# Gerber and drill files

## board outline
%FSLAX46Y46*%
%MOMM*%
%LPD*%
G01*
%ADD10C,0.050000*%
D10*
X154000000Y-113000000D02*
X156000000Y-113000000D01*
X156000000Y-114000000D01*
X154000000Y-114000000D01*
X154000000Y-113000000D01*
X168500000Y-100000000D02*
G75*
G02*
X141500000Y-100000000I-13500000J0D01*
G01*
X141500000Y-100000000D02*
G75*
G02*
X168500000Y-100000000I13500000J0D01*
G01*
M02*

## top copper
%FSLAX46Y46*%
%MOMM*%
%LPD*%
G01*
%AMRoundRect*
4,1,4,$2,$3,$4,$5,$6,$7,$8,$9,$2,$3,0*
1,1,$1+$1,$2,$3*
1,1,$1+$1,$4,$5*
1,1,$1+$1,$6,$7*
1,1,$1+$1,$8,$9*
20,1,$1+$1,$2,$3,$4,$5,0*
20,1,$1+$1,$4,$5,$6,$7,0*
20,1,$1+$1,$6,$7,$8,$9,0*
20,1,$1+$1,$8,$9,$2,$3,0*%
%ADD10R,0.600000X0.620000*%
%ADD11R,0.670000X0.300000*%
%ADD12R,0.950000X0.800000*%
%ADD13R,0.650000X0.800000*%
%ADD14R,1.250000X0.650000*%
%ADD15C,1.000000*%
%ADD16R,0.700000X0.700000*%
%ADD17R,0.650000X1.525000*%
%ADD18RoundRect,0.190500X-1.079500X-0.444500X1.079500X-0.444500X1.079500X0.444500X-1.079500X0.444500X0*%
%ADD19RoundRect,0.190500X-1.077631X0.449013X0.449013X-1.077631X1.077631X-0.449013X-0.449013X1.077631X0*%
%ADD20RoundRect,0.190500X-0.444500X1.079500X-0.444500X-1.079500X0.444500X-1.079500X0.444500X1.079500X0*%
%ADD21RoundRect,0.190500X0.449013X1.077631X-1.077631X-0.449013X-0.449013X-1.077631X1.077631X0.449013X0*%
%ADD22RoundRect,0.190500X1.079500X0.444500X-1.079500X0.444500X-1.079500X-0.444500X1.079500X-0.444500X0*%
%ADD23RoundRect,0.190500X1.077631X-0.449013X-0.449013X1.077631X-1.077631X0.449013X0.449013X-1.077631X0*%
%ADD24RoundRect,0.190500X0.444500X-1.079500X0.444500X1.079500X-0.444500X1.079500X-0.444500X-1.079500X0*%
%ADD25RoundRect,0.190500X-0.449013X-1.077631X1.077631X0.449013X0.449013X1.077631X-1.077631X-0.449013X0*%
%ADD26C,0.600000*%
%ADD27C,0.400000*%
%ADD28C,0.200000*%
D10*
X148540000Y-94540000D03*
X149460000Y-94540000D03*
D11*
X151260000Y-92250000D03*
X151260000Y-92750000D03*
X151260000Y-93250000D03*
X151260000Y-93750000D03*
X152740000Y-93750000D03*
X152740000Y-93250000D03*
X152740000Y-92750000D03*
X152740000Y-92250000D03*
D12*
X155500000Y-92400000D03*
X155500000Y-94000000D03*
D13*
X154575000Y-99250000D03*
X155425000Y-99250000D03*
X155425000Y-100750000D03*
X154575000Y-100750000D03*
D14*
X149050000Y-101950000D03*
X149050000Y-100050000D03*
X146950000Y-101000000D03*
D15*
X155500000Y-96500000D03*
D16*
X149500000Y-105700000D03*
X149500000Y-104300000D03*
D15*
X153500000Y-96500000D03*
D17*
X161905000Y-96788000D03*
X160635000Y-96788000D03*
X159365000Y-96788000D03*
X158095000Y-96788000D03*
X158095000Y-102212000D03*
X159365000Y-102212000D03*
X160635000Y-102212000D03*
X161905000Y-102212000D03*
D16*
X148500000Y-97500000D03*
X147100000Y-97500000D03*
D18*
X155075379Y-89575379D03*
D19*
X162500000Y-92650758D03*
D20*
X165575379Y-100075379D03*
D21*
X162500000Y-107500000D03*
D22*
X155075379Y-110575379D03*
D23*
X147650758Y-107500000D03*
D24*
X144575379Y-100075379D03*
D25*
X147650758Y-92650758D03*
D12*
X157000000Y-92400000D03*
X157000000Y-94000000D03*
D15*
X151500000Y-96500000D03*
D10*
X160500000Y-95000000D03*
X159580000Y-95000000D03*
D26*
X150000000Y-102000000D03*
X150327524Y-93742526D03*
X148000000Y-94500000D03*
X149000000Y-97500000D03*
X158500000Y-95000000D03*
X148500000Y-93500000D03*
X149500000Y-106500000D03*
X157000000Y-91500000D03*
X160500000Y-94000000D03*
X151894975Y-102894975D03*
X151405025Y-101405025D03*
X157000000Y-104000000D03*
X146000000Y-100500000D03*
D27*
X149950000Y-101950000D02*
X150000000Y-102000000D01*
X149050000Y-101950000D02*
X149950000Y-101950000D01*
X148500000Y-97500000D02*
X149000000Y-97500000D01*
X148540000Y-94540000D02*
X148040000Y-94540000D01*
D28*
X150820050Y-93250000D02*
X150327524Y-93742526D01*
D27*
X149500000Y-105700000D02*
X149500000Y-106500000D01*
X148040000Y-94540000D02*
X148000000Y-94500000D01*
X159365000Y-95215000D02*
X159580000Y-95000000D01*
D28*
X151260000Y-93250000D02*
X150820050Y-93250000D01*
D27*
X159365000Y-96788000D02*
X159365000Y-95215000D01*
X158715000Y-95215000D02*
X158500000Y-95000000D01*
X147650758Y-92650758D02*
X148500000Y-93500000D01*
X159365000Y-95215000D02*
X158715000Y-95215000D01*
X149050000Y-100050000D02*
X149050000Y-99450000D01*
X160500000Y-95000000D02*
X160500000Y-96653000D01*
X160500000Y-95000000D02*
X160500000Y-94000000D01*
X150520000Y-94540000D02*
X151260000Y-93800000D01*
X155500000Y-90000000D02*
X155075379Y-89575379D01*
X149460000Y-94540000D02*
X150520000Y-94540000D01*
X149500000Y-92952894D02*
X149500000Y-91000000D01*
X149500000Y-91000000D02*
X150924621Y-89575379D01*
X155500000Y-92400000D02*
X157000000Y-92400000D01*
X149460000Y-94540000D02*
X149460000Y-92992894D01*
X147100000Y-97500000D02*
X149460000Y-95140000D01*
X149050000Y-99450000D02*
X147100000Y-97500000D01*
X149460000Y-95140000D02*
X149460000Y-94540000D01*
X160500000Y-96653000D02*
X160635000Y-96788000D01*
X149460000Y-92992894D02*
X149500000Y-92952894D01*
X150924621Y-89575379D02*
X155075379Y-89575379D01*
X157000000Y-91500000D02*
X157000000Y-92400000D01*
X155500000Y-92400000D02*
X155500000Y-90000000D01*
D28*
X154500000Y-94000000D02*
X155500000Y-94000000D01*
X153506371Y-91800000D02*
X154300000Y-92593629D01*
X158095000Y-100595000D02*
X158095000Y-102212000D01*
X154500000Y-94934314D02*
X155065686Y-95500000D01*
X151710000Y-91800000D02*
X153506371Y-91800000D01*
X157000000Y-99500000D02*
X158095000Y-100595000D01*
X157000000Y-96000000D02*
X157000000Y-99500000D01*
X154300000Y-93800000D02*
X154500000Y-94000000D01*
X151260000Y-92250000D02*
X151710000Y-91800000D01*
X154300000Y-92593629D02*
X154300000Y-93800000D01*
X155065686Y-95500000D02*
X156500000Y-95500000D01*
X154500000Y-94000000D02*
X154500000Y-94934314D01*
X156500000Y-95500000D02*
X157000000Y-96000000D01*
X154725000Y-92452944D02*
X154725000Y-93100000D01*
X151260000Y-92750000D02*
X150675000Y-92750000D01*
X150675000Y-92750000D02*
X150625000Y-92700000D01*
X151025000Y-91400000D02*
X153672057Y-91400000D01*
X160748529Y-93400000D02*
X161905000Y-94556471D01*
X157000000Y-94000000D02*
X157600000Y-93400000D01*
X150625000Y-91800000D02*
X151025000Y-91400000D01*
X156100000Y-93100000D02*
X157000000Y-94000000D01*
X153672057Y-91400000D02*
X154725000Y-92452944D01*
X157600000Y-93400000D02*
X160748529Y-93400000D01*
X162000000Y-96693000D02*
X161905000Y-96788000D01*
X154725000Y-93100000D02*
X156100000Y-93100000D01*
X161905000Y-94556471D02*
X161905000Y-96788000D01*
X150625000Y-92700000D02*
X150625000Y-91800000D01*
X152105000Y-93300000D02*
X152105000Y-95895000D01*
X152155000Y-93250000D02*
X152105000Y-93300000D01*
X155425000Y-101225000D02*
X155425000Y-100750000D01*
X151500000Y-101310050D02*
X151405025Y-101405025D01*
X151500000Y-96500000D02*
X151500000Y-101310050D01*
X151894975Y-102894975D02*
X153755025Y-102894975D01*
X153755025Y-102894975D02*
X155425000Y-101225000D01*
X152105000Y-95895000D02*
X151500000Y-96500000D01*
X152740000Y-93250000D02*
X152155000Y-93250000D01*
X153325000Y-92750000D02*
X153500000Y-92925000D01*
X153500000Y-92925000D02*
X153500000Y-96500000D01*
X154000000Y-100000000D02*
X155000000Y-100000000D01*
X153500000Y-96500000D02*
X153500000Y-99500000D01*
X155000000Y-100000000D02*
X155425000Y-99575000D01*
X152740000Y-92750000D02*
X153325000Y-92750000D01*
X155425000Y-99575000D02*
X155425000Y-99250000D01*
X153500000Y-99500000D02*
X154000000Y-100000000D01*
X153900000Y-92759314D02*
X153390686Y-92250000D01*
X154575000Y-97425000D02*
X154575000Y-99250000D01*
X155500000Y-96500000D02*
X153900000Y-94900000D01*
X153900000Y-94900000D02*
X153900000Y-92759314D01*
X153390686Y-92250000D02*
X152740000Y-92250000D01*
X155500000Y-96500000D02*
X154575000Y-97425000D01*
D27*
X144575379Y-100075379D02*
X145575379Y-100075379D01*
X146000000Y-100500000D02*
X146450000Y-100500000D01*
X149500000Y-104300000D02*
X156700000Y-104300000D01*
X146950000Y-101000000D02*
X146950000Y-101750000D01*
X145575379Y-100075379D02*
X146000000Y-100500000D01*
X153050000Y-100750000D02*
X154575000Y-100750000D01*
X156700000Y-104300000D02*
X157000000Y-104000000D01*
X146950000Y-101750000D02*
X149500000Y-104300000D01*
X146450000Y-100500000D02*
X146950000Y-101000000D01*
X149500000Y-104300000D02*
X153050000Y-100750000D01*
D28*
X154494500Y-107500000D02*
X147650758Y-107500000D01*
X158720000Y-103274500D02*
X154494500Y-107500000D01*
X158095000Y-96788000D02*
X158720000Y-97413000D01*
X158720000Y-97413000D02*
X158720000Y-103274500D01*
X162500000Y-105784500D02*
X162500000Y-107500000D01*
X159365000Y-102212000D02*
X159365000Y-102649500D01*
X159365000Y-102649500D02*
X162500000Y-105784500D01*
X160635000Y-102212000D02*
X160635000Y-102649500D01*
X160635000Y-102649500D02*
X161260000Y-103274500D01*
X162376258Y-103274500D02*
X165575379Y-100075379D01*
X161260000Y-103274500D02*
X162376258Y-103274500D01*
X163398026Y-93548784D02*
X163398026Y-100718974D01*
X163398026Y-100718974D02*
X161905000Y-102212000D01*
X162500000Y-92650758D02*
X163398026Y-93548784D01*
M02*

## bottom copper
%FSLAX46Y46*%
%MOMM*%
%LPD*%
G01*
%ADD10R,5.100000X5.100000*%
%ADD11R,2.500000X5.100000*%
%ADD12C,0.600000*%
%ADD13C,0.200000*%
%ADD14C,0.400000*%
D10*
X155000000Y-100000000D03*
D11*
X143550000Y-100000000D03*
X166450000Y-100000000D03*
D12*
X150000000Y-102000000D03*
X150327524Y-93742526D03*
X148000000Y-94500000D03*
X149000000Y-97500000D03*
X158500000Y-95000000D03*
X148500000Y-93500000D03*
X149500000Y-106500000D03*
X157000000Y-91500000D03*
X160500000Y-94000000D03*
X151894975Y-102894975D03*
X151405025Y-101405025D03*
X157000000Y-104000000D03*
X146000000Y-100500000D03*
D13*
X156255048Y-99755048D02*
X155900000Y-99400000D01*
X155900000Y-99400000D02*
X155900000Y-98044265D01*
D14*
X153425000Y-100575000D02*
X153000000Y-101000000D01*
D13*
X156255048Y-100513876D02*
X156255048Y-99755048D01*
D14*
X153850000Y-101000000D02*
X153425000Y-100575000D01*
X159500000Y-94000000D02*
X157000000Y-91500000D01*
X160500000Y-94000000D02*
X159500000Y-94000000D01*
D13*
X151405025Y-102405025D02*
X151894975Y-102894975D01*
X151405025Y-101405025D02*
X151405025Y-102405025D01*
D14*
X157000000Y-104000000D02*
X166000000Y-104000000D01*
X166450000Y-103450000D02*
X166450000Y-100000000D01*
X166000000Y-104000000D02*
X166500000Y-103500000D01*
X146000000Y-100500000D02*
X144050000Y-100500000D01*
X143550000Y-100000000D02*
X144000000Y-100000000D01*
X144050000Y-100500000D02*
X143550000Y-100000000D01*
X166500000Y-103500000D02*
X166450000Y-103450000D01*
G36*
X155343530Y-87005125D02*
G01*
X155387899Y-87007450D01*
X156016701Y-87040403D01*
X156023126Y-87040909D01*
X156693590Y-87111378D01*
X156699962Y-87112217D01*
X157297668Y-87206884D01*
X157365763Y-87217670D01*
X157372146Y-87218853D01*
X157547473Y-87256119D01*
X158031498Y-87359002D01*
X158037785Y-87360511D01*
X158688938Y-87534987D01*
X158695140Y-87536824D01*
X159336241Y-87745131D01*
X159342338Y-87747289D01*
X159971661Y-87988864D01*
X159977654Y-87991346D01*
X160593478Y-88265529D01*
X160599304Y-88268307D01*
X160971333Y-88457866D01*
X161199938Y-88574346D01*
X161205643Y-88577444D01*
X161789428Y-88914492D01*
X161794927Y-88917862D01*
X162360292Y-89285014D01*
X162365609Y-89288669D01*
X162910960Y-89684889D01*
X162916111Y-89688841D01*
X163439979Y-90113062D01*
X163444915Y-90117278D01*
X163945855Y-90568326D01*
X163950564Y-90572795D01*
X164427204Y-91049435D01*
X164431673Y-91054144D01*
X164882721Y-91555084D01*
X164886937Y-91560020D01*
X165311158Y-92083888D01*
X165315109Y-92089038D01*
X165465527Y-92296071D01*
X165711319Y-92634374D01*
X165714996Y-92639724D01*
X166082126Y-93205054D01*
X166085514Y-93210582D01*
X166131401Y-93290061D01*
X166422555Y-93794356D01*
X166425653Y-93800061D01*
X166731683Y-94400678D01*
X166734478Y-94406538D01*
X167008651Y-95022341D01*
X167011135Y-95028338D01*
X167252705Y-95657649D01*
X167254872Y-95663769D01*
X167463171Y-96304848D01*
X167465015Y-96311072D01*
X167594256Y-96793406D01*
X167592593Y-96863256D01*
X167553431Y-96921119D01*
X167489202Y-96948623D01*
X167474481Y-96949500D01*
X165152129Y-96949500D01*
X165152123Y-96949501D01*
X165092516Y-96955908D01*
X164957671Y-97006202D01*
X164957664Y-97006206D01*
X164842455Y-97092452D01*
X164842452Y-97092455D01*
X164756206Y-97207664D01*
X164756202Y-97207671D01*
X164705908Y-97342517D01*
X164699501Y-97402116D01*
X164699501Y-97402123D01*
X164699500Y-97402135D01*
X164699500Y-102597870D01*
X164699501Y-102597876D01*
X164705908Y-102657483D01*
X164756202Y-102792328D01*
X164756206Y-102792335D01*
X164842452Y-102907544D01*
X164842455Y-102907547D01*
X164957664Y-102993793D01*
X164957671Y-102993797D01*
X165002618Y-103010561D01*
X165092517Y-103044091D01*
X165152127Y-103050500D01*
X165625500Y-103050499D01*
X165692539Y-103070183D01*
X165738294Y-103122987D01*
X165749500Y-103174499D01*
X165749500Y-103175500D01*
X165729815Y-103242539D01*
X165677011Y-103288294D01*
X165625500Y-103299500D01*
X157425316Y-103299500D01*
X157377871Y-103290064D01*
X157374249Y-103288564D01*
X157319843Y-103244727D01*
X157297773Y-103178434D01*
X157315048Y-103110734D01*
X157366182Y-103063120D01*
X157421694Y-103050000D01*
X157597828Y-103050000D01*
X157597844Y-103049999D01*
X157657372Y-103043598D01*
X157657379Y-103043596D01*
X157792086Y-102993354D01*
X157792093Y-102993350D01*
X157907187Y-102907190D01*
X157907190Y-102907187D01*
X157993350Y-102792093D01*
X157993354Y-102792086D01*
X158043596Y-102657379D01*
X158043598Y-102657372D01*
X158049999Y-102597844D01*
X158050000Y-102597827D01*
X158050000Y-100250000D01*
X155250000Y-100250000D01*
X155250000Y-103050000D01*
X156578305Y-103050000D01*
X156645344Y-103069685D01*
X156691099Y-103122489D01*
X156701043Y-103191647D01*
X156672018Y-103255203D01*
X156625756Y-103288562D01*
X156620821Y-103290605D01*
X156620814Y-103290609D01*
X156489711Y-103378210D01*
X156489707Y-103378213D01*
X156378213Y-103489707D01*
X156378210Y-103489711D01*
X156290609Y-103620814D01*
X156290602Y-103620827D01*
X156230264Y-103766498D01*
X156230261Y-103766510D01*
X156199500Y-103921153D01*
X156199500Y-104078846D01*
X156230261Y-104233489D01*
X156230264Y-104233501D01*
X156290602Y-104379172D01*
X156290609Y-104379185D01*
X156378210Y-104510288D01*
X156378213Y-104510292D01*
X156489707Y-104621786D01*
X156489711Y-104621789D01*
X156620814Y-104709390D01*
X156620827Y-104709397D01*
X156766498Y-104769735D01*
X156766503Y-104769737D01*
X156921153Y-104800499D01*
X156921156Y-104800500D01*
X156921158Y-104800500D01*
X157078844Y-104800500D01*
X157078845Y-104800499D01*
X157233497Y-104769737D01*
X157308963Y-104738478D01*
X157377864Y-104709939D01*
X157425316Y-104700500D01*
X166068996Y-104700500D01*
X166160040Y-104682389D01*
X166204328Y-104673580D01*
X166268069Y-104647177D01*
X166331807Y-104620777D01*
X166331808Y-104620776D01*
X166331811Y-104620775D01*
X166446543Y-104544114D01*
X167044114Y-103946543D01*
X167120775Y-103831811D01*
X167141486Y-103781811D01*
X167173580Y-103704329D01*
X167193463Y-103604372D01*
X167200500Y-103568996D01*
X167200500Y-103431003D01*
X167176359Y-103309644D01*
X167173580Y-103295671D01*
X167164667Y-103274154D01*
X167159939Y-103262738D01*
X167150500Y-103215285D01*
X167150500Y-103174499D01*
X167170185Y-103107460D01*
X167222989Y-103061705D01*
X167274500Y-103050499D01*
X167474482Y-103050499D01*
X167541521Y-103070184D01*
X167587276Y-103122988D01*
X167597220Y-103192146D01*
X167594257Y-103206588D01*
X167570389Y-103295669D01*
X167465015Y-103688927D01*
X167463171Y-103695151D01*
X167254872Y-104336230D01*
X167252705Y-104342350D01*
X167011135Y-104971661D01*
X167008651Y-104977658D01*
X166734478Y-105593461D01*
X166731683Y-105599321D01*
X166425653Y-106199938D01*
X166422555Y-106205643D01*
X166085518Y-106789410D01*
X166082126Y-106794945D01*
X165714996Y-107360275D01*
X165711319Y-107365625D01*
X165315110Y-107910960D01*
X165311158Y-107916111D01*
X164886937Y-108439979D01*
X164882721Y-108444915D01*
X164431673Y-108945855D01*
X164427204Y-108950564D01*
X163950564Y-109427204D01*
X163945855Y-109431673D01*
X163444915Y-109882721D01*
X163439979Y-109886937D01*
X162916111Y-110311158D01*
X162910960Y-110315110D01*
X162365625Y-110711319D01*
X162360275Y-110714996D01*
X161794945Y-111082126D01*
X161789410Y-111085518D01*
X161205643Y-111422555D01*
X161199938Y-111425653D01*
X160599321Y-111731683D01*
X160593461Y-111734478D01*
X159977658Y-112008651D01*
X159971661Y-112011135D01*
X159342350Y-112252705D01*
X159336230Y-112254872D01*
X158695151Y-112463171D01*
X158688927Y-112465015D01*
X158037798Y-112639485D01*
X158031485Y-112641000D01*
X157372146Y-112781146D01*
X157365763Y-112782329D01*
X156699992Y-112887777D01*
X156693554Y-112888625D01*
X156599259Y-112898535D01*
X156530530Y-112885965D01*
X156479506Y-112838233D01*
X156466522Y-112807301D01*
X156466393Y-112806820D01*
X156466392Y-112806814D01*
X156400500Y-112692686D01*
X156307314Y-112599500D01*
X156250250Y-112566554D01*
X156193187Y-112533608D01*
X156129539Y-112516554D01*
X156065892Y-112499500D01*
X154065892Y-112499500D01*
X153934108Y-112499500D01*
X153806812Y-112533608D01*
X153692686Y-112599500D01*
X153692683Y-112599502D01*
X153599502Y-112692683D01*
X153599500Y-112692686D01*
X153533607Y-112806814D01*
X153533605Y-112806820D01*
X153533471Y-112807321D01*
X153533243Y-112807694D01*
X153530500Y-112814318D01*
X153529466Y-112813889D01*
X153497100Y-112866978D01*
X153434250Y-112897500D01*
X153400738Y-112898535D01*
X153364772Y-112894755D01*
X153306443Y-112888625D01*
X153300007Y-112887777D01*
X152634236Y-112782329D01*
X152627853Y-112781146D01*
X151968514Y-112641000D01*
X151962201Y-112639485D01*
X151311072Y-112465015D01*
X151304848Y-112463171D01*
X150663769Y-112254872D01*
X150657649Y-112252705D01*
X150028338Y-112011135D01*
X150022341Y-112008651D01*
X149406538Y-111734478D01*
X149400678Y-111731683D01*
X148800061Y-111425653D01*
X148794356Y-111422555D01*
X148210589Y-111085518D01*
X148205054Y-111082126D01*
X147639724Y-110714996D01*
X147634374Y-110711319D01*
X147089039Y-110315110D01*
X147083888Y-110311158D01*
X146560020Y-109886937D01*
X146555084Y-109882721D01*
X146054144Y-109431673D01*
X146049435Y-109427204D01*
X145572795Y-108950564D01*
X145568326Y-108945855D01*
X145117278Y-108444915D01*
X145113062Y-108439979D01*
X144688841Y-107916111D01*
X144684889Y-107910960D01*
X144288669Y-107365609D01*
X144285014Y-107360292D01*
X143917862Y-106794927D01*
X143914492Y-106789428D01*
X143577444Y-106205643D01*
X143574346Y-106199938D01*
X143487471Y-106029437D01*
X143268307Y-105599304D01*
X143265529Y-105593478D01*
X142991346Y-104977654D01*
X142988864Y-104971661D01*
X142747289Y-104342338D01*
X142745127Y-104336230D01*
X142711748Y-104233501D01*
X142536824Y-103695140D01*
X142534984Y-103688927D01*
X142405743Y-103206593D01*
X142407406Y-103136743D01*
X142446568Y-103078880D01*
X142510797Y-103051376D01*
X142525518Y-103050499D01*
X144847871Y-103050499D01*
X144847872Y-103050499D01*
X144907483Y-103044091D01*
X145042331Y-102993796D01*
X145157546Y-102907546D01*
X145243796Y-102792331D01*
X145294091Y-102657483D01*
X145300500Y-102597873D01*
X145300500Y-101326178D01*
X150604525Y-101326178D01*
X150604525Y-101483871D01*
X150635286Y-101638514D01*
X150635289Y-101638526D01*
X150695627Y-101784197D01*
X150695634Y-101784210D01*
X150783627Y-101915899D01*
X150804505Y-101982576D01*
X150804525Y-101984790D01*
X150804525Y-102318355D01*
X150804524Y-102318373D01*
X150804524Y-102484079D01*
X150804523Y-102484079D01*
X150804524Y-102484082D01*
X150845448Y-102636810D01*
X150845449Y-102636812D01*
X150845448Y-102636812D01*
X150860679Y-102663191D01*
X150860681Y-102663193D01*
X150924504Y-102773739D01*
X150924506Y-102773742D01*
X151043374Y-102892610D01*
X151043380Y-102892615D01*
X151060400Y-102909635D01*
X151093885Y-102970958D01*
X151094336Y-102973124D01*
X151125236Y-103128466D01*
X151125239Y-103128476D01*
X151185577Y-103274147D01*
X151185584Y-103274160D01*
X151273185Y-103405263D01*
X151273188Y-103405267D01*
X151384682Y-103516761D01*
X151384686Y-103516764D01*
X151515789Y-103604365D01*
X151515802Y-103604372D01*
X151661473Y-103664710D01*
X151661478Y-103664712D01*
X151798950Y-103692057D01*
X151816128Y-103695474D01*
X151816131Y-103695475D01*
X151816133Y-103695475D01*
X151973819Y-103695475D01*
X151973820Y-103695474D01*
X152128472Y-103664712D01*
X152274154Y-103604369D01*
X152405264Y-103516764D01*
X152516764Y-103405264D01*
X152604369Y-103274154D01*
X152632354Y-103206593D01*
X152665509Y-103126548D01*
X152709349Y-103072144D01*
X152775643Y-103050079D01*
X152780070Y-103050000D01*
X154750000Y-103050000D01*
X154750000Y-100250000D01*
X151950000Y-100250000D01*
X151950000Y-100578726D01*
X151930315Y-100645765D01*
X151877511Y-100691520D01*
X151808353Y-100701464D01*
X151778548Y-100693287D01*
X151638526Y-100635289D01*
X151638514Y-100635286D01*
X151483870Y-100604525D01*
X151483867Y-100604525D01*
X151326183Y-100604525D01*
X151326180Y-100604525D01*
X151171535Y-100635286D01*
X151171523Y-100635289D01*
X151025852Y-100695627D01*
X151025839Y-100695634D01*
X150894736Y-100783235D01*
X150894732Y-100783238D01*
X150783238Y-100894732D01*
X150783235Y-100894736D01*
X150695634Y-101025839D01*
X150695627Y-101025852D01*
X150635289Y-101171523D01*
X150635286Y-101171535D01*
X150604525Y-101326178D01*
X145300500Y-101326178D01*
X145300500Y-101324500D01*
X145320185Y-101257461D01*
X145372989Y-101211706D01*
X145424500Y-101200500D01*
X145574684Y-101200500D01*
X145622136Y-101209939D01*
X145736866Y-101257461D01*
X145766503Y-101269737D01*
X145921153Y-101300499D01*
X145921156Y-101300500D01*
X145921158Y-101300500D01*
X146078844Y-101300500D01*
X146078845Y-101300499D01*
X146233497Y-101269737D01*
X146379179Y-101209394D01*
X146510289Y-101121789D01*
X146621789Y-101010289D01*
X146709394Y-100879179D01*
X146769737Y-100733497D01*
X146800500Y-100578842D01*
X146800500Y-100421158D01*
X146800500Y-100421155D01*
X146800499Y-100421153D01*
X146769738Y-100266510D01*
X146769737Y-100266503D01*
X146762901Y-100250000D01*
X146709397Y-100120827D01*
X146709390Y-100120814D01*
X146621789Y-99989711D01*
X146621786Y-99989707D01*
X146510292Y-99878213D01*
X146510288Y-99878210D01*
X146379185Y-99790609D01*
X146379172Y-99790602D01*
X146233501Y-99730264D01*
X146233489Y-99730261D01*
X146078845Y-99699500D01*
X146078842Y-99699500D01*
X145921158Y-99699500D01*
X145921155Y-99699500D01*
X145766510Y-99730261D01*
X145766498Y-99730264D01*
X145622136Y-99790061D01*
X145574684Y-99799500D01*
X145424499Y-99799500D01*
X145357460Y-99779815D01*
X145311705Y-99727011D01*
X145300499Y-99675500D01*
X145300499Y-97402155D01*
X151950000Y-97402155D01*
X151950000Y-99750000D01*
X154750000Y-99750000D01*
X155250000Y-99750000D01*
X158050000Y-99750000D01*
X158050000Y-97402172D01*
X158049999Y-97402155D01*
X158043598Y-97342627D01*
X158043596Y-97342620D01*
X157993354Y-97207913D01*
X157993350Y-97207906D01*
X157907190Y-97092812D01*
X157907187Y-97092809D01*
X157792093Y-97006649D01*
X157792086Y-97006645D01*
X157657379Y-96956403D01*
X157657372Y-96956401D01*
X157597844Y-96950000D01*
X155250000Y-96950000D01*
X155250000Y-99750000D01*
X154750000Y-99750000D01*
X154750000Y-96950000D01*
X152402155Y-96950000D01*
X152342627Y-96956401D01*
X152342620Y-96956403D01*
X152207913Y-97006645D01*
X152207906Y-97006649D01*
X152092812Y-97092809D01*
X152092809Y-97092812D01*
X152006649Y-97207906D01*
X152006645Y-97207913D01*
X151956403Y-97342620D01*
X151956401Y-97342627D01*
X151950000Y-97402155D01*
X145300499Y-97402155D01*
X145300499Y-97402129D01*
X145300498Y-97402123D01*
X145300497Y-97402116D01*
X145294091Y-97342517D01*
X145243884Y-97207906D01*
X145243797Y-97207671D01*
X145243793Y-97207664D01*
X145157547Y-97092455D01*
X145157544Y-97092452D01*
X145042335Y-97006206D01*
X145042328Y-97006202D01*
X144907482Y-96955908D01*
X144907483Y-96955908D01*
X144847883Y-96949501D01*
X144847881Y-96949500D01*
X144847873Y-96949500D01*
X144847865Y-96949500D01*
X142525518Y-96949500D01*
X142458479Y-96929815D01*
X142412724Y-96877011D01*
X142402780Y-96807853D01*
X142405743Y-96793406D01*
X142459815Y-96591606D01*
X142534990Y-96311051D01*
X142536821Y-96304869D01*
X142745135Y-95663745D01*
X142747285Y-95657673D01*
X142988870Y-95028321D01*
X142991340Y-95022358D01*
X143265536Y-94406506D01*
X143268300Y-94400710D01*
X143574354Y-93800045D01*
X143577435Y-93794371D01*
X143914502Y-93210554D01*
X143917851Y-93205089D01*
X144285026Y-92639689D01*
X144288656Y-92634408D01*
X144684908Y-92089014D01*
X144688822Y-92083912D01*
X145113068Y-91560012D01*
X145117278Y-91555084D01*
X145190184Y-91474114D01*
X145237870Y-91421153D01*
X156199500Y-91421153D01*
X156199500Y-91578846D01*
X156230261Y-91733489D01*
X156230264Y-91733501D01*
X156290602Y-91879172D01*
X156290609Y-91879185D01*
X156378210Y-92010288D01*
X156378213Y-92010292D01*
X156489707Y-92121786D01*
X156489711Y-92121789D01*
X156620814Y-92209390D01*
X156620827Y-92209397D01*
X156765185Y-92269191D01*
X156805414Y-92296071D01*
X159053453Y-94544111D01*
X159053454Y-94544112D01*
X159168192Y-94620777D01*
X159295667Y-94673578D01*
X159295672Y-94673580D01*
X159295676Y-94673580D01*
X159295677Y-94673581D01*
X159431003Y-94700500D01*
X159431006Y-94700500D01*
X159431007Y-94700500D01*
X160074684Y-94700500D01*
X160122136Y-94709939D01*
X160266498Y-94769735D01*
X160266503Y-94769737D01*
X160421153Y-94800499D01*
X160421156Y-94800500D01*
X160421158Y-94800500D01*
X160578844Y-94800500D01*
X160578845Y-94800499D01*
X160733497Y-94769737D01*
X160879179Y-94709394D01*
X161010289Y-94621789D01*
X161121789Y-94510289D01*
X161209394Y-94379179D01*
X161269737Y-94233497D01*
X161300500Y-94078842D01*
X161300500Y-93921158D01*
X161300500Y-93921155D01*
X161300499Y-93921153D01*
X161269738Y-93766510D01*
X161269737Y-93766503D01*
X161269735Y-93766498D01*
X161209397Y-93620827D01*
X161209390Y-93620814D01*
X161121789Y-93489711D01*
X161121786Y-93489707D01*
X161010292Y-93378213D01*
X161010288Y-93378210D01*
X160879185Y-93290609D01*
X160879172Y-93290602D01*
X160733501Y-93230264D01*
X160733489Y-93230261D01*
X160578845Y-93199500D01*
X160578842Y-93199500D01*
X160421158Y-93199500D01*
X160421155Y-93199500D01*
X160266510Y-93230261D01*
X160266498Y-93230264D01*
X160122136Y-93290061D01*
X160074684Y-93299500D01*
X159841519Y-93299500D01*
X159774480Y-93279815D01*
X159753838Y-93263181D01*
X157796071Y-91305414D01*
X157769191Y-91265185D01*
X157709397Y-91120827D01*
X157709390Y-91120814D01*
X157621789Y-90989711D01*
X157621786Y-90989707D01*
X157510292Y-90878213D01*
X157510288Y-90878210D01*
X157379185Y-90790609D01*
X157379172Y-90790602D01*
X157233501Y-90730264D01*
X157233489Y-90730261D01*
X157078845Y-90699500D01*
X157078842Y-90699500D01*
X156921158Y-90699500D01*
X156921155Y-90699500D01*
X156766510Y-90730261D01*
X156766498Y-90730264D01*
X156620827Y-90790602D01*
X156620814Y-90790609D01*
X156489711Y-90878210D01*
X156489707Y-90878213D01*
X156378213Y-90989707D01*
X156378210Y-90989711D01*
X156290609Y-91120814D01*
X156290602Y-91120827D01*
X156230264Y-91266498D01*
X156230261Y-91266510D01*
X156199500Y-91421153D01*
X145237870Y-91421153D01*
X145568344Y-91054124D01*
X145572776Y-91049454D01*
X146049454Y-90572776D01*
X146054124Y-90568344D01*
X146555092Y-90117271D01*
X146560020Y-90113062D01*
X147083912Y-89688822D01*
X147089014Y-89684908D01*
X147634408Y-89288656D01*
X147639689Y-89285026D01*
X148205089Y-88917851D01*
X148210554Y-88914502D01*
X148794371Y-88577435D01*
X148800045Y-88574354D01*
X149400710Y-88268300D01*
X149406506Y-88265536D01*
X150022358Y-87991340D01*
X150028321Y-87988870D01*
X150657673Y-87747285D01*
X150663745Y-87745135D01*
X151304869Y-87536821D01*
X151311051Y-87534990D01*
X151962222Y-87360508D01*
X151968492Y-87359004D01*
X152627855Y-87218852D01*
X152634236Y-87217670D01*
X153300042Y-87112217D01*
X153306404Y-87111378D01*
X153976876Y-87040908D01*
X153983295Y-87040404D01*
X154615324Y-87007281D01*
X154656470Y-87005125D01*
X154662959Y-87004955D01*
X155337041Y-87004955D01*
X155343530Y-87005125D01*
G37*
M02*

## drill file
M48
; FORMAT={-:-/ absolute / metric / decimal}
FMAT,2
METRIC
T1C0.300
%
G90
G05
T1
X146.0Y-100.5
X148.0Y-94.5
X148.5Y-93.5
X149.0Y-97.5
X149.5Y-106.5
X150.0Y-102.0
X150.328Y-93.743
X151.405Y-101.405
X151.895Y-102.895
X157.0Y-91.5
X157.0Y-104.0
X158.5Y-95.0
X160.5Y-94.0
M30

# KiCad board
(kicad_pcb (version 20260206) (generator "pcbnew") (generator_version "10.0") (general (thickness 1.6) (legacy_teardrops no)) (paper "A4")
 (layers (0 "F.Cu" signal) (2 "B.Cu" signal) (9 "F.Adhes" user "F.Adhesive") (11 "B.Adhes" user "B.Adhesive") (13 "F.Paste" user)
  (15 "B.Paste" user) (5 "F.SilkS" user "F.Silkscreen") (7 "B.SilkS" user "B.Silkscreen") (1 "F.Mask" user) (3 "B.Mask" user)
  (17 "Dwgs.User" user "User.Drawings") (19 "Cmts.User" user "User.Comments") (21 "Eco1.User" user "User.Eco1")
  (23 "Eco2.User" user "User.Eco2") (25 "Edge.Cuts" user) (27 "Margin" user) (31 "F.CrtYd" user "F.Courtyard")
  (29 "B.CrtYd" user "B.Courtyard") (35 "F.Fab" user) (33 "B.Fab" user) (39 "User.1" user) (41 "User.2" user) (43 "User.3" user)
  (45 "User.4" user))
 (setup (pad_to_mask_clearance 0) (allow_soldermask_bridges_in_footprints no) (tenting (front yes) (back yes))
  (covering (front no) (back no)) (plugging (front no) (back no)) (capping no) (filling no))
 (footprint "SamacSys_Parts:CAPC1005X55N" (layer "F.Cu") (at 149 94.54)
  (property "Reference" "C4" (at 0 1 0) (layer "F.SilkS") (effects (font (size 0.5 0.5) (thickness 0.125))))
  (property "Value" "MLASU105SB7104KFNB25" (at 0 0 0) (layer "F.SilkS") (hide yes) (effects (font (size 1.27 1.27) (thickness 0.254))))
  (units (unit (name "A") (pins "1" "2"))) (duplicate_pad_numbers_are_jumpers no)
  (pad "1" smd rect (at -0.46 0) (size 0.6 0.62) (layers "F.Cu" "F.Mask" "F.Paste") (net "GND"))
  (pad "2" smd rect (at 0.46 0) (size 0.6 0.62) (layers "F.Cu" "F.Mask" "F.Paste") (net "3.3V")))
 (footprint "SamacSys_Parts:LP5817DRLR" (layer "F.Cu") (at 152 93)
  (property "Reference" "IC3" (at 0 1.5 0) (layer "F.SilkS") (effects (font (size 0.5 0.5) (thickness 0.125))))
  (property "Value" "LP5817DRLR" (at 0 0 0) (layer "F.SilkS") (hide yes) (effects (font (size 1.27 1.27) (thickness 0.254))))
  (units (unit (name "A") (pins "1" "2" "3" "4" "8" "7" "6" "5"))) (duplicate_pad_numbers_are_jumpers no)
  (pad "1" smd rect (at -0.74 -0.75 90) (size 0.3 0.67) (layers "F.Cu" "F.Mask" "F.Paste") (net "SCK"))
  (pad "2" smd rect (at -0.74 -0.25 90) (size 0.3 0.67) (layers "F.Cu" "F.Mask" "F.Paste") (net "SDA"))
  (pad "3" smd rect (at -0.74 0.25 90) (size 0.3 0.67) (layers "F.Cu" "F.Mask" "F.Paste") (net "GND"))
  (pad "4" smd rect (at -0.74 0.75 90) (size 0.3 0.67) (layers "F.Cu" "F.Mask" "F.Paste") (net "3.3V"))
  (pad "5" smd rect (at 0.74 0.75 90) (size 0.3 0.67) (layers "F.Cu" "F.Mask" "F.Paste") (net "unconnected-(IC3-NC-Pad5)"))
  (pad "6" smd rect (at 0.74 0.25 90) (size 0.3 0.67) (layers "F.Cu" "F.Mask" "F.Paste") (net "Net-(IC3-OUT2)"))
  (pad "7" smd rect (at 0.74 -0.25 90) (size 0.3 0.67) (layers "F.Cu" "F.Mask" "F.Paste") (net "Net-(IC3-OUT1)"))
  (pad "8" smd rect (at 0.74 -0.75 90) (size 0.3 0.67) (layers "F.Cu" "F.Mask" "F.Paste") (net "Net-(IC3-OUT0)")))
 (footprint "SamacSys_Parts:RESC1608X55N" (layer "F.Cu") (at 155.5 93.2 -90)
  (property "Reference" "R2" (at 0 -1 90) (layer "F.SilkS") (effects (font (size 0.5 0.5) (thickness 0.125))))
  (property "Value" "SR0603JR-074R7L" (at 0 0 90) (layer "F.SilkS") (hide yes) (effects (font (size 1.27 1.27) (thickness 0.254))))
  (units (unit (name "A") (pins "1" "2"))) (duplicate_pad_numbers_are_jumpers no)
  (pad "1" smd rect (at -0.8 0 270) (size 0.8 0.95) (layers "F.Cu" "F.Mask" "F.Paste") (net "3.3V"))
  (pad "2" smd rect (at 0.8 0 270) (size 0.8 0.95) (layers "F.Cu" "F.Mask" "F.Paste") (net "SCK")))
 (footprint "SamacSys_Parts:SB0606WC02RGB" (layer "F.Cu") (at 155 100 90)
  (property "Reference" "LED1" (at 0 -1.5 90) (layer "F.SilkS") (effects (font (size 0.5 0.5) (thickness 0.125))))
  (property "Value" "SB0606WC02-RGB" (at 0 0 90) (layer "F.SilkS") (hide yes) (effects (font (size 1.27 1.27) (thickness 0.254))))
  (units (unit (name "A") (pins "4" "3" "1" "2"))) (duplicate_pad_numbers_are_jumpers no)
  (pad "1" smd rect (at 0.75 -0.425 180) (size 0.65 0.8) (layers "F.Cu" "F.Mask" "F.Paste") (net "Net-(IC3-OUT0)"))
  (pad "2" smd rect (at 0.75 0.425 180) (size 0.65 0.8) (layers "F.Cu" "F.Mask" "F.Paste") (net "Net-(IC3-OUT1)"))
  (pad "3" smd rect (at -0.75 0.425 180) (size 0.65 0.8) (layers "F.Cu" "F.Mask" "F.Paste") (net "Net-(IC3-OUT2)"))
  (pad "4" smd rect (at -0.75 -0.425 180) (size 0.65 0.8) (layers "F.Cu" "F.Mask" "F.Paste") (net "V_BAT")))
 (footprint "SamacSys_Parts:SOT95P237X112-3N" (layer "F.Cu") (at 148 101 180)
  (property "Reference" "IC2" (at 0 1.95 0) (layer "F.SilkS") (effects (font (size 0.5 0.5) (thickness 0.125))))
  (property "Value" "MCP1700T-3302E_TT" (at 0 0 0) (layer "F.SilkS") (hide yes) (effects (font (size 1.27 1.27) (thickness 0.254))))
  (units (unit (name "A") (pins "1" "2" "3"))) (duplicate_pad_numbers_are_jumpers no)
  (pad "1" smd rect (at -1.05 -0.95 270) (size 0.65 1.25) (layers "F.Cu" "F.Mask" "F.Paste") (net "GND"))
  (pad "2" smd rect (at -1.05 0.95 270) (size 0.65 1.25) (layers "F.Cu" "F.Mask" "F.Paste") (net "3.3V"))
  (pad "3" smd rect (at 1.05 0 270) (size 0.65 1.25) (layers "F.Cu" "F.Mask" "F.Paste") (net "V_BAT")))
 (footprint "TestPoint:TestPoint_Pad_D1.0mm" (layer "F.Cu") (at 155.5 96.5 90)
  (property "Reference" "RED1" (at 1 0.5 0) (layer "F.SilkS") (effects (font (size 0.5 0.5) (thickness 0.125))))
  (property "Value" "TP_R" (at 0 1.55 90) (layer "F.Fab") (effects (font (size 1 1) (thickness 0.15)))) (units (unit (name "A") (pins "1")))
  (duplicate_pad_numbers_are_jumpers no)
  (pad "1" smd circle (at 0 0 90) (size 1 1) (layers "F.Cu" "F.Mask") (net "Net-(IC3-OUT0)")))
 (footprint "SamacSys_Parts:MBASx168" (layer "F.Cu") (at 149.5 105 90)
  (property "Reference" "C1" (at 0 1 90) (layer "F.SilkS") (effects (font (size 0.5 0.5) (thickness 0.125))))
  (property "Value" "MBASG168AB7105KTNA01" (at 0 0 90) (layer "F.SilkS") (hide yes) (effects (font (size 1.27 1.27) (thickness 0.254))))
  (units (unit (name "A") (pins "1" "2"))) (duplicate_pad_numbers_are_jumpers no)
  (pad "1" smd rect (at -0.7 0 90) (size 0.7 0.7) (layers "F.Cu" "F.Mask" "F.Paste") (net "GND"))
  (pad "2" smd rect (at 0.7 0 90) (size 0.7 0.7) (layers "F.Cu" "F.Mask" "F.Paste") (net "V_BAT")))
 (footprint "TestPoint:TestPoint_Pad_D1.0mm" (layer "F.Cu") (at 153.5 96.5 90)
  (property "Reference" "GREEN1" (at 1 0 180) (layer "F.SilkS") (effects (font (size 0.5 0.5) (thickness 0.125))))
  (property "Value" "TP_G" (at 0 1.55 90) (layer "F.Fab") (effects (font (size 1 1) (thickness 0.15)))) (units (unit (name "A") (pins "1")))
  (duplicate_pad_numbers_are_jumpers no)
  (pad "1" smd circle (at 0 0 90) (size 1 1) (layers "F.Cu" "F.Mask") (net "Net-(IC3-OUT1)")))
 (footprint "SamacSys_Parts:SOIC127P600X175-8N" (layer "F.Cu") (at 160 99.5 -90)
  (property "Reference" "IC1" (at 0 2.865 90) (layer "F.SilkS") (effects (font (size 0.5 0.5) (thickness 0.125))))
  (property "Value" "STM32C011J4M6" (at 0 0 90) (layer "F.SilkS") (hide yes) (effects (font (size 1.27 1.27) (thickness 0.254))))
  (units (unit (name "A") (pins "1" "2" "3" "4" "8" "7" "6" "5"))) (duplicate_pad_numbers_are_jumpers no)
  (pad "1" smd rect (at -2.712 -1.905) (size 0.65 1.525) (layers "F.Cu" "F.Mask" "F.Paste") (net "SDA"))
  (pad "2" smd rect (at -2.712 -0.635) (size 0.65 1.525) (layers "F.Cu" "F.Mask" "F.Paste") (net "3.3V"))
  (pad "3" smd rect (at -2.712 0.635) (size 0.65 1.525) (layers "F.Cu" "F.Mask" "F.Paste") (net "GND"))
  (pad "4" smd rect (at -2.712 1.905) (size 0.65 1.525) (layers "F.Cu" "F.Mask" "F.Paste") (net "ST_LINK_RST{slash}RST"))
  (pad "5" smd rect (at 2.712 1.905) (size 0.65 1.525) (layers "F.Cu" "F.Mask" "F.Paste") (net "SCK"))
  (pad "6" smd rect (at 2.712 0.635) (size 0.65 1.525) (layers "F.Cu" "F.Mask" "F.Paste") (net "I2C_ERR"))
  (pad "7" smd rect (at 2.712 -0.635) (size 0.65 1.525) (layers "F.Cu" "F.Mask" "F.Paste") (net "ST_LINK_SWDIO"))
  (pad "8" smd rect (at 2.712 -1.905) (size 0.65 1.525) (layers "F.Cu" "F.Mask" "F.Paste") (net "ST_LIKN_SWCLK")))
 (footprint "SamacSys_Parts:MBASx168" (layer "F.Cu") (at 147.8 97.5 180)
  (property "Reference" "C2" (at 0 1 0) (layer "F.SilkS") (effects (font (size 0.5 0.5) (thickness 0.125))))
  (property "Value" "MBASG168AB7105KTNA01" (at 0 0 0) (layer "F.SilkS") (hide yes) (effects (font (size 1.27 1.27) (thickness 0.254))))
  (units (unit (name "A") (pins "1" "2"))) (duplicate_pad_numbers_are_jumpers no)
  (pad "1" smd rect (at -0.7 0 180) (size 0.7 0.7) (layers "F.Cu" "F.Mask" "F.Paste") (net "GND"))
  (pad "2" smd rect (at 0.7 0 180) (size 0.7 0.7) (layers "F.Cu" "F.Mask" "F.Paste") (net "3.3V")))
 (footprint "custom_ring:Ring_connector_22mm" (layer "F.Cu") (at 155.075379 89.575379)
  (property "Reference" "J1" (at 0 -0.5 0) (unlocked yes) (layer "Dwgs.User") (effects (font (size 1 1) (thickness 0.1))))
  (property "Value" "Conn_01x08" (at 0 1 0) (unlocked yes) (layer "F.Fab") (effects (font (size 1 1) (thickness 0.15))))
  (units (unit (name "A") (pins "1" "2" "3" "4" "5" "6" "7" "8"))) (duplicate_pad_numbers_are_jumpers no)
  (pad "1" smd roundrect (at 0 0) (size 2.54 1.27) (layers "F.Cu" "F.Mask" "F.Paste") (roundrect_rratio 0.15) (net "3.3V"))
  (pad "2" smd roundrect (at 7.424621 3.075379 315) (size 2.54 1.27) (layers "F.Cu" "F.Mask" "F.Paste") (roundrect_rratio 0.15)
   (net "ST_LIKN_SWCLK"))
  (pad "3" smd roundrect (at 10.5 10.5 270) (size 2.54 1.27) (layers "F.Cu" "F.Mask" "F.Paste") (roundrect_rratio 0.15)
   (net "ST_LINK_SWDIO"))
  (pad "4" smd roundrect (at 7.424621 17.924621 225) (size 2.54 1.27) (layers "F.Cu" "F.Mask" "F.Paste") (roundrect_rratio 0.15)
   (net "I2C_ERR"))
  (pad "5" smd roundrect (at 0 21 180) (size 2.54 1.27) (layers "F.Cu" "F.Mask" "F.Paste") (roundrect_rratio 0.15)
   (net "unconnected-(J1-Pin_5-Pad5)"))
  (pad "6" smd roundrect (at -7.424621 17.924621 135) (size 2.54 1.27) (layers "F.Cu" "F.Mask" "F.Paste") (roundrect_rratio 0.15)
   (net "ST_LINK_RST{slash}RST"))
  (pad "7" smd roundrect (at -10.5 10.5 90) (size 2.54 1.27) (layers "F.Cu" "F.Mask" "F.Paste") (roundrect_rratio 0.15) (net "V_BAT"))
  (pad "8" smd roundrect (at -7.424621 3.075379 45) (size 2.54 1.27) (layers "F.Cu" "F.Mask" "F.Paste") (roundrect_rratio 0.15) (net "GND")))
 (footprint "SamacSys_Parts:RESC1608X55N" (layer "F.Cu") (at 157 93.2 -90)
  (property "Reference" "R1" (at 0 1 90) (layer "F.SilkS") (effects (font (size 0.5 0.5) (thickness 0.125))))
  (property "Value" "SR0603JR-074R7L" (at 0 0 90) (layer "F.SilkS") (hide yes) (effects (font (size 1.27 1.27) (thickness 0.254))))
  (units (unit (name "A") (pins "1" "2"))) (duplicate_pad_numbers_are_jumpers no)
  (pad "1" smd rect (at -0.8 0 270) (size 0.8 0.95) (layers "F.Cu" "F.Mask" "F.Paste") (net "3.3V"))
  (pad "2" smd rect (at 0.8 0 270) (size 0.8 0.95) (layers "F.Cu" "F.Mask" "F.Paste") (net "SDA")))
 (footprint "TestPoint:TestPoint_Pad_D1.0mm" (layer "F.Cu") (at 151.5 96.5 90)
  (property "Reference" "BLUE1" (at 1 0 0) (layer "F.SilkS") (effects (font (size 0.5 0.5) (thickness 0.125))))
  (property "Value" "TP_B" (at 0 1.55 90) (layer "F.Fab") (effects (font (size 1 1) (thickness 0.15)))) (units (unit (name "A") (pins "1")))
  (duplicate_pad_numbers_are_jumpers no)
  (pad "1" smd circle (at 0 0 90) (size 1 1) (layers "F.Cu" "F.Mask") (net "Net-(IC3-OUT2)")))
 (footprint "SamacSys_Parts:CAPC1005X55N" (layer "F.Cu") (at 160.04 95 180)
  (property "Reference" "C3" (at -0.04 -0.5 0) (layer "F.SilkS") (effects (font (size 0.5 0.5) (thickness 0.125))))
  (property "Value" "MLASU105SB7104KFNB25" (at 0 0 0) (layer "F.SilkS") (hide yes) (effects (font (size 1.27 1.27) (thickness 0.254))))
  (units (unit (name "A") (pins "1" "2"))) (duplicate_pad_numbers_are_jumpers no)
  (pad "1" smd rect (at -0.46 0 180) (size 0.6 0.62) (layers "F.Cu" "F.Mask" "F.Paste") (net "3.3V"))
  (pad "2" smd rect (at 0.46 0 180) (size 0.6 0.62) (layers "F.Cu" "F.Mask" "F.Paste") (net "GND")))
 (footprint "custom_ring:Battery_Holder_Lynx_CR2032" (layer "B.Cu") (at 155 100 180)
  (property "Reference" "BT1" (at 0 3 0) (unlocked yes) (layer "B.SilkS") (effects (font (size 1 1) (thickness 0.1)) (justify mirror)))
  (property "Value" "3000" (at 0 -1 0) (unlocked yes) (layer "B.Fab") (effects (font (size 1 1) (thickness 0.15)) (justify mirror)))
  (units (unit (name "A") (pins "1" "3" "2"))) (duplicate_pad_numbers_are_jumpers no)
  (pad "1" smd rect (at 0 0 180) (size 5.1 5.1) (layers "B.Cu" "B.Mask" "B.Paste") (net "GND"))
  (pad "2" smd rect (at 11.45 0 180) (size 2.5 5.1) (layers "B.Cu" "B.Mask" "B.Paste") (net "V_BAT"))
  (pad "3" smd rect (at -11.45 0 180) (size 2.5 5.1) (layers "B.Cu" "B.Mask" "B.Paste") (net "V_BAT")))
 (gr_rect (start 154 113) (end 156 114) (stroke (width 0.05) (type default)) (fill no) (layer "Edge.Cuts"))
 (gr_circle (center 155 100) (end 168.5 100) (stroke (width 0.05) (type solid)) (fill no) (layer "Edge.Cuts"))
 (segment (start 149.95 101.95) (end 150 102) (width 0.4) (layer "F.Cu") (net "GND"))
 (segment (start 149.05 101.95) (end 149.95 101.95) (width 0.4) (layer "F.Cu") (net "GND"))
 (segment (start 148.5 97.5) (end 149 97.5) (width 0.4) (layer "F.Cu") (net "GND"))
 (segment (start 148.54 94.54) (end 148.04 94.54) (width 0.4) (layer "F.Cu") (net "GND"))
 (segment (start 150.82005 93.25) (end 150.327524 93.742526) (width 0.2) (layer "F.Cu") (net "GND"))
 (segment (start 149.5 105.7) (end 149.5 106.5) (width 0.4) (layer "F.Cu") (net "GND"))
 (segment (start 148.04 94.54) (end 148 94.5) (width 0.4) (layer "F.Cu") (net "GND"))
 (segment (start 159.365 95.215) (end 159.58 95) (width 0.4) (layer "F.Cu") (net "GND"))
 (segment (start 151.26 93.25) (end 150.82005 93.25) (width 0.2) (layer "F.Cu") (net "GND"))
 (segment (start 159.365 96.788) (end 159.365 95.215) (width 0.4) (layer "F.Cu") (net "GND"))
 (segment (start 158.715 95.215) (end 158.5 95) (width 0.4) (layer "F.Cu") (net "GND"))
 (segment (start 147.650758 92.650758) (end 148.5 93.5) (width 0.4) (layer "F.Cu") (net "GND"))
 (segment (start 159.365 95.215) (end 158.715 95.215) (width 0.4) (layer "F.Cu") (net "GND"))
 (via (at 150 102) (size 0.6) (drill 0.3) (layers "F.Cu" "B.Cu") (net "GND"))
 (via (at 150.327524 93.742526) (size 0.6) (drill 0.3) (layers "F.Cu" "B.Cu") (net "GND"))
 (via (at 148 94.5) (size 0.6) (drill 0.3) (layers "F.Cu" "B.Cu") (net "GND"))
 (via (at 149 97.5) (size 0.6) (drill 0.3) (layers "F.Cu" "B.Cu") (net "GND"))
 (via (at 158.5 95) (size 0.6) (drill 0.3) (layers "F.Cu" "B.Cu") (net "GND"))
 (via (at 148.5 93.5) (size 0.6) (drill 0.3) (layers "F.Cu" "B.Cu") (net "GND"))
 (via (at 149.5 106.5) (size 0.6) (drill 0.3) (layers "F.Cu" "B.Cu") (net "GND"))
 (segment (start 156.255048 99.755048) (end 155.9 99.4) (width 0.2) (layer "B.Cu") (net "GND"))
 (segment (start 155.9 99.4) (end 155.9 98.044265) (width 0.2) (layer "B.Cu") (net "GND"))
 (segment (start 153.425 100.575) (end 153 101) (width 0.4) (layer "B.Cu") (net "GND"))
 (segment (start 156.255048 100.513876) (end 156.255048 99.755048) (width 0.2) (layer "B.Cu") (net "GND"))
 (segment (start 153.85 101) (end 153.425 100.575) (width 0.4) (layer "B.Cu") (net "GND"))
 (segment (start 149.05 100.05) (end 149.05 99.45) (width 0.4) (layer "F.Cu") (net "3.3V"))
 (segment (start 160.5 95) (end 160.5 96.653) (width 0.4) (layer "F.Cu") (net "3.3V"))
 (segment (start 160.5 95) (end 160.5 94) (width 0.4) (layer "F.Cu") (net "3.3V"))
 (segment (start 150.52 94.54) (end 151.26 93.8) (width 0.4) (layer "F.Cu") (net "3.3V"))
 (segment (start 155.5 90) (end 155.075379 89.575379) (width 0.4) (layer "F.Cu") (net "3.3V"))
 (segment (start 149.46 94.54) (end 150.52 94.54) (width 0.4) (layer "F.Cu") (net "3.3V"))
 (segment (start 149.5 92.952894) (end 149.5 91) (width 0.4) (layer "F.Cu") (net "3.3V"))
 (segment (start 149.5 91) (end 150.924621 89.575379) (width 0.4) (layer "F.Cu") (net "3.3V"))
 (segment (start 155.5 92.4) (end 157 92.4) (width 0.4) (layer "F.Cu") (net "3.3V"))
 (segment (start 149.46 94.54) (end 149.46 92.992894) (width 0.4) (layer "F.Cu") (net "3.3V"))
 (segment (start 147.1 97.5) (end 149.46 95.14) (width 0.4) (layer "F.Cu") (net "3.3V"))
 (segment (start 149.05 99.45) (end 147.1 97.5) (width 0.4) (layer "F.Cu") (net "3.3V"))
 (segment (start 149.46 95.14) (end 149.46 94.54) (width 0.4) (layer "F.Cu") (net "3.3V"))
 (segment (start 160.5 96.653) (end 160.635 96.788) (width 0.4) (layer "F.Cu") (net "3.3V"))
 (segment (start 149.46 92.992894) (end 149.5 92.952894) (width 0.4) (layer "F.Cu") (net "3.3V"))
 (segment (start 150.924621 89.575379) (end 155.075379 89.575379) (width 0.4) (layer "F.Cu") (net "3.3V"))
 (segment (start 157 91.5) (end 157 92.4) (width 0.4) (layer "F.Cu") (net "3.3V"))
 (segment (start 155.5 92.4) (end 155.5 90) (width 0.4) (layer "F.Cu") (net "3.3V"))
 (via (at 157 91.5) (size 0.6) (drill 0.3) (layers "F.Cu" "B.Cu") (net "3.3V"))
 (via (at 160.5 94) (size 0.6) (drill 0.3) (layers "F.Cu" "B.Cu") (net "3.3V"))
 (segment (start 159.5 94) (end 157 91.5) (width 0.4) (layer "B.Cu") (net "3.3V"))
 (segment (start 160.5 94) (end 159.5 94) (width 0.4) (layer "B.Cu") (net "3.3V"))
 (segment (start 154.5 94) (end 155.5 94) (width 0.2) (layer "F.Cu") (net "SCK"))
 (segment (start 153.506371 91.8) (end 154.3 92.593629) (width 0.2) (layer "F.Cu") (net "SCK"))
 (segment (start 158.095 100.595) (end 158.095 102.212) (width 0.2) (layer "F.Cu") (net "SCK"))
 (segment (start 154.5 94.934314) (end 155.065686 95.5) (width 0.2) (layer "F.Cu") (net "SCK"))
 (segment (start 151.71 91.8) (end 153.506371 91.8) (width 0.2) (layer "F.Cu") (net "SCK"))
 (segment (start 157 99.5) (end 158.095 100.595) (width 0.2) (layer "F.Cu") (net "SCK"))
 (segment (start 157 96) (end 157 99.5) (width 0.2) (layer "F.Cu") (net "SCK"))
 (segment (start 154.3 93.8) (end 154.5 94) (width 0.2) (layer "F.Cu") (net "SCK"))
 (segment (start 151.26 92.25) (end 151.71 91.8) (width 0.2) (layer "F.Cu") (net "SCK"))
 (segment (start 154.3 92.593629) (end 154.3 93.8) (width 0.2) (layer "F.Cu") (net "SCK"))
 (segment (start 155.065686 95.5) (end 156.5 95.5) (width 0.2) (layer "F.Cu") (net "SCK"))
 (segment (start 154.5 94) (end 154.5 94.934314) (width 0.2) (layer "F.Cu") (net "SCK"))
 (segment (start 156.5 95.5) (end 157 96) (width 0.2) (layer "F.Cu") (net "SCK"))
 (segment (start 154.725 92.452944) (end 154.725 93.1) (width 0.2) (layer "F.Cu") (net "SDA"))
 (segment (start 151.26 92.75) (end 150.675 92.75) (width 0.2) (layer "F.Cu") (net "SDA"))
 (segment (start 150.675 92.75) (end 150.625 92.7) (width 0.2) (layer "F.Cu") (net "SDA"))
 (segment (start 151.025 91.4) (end 153.672057 91.4) (width 0.2) (layer "F.Cu") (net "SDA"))
 (segment (start 160.748529 93.4) (end 161.905 94.556471) (width 0.2) (layer "F.Cu") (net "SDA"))
 (segment (start 157 94) (end 157.6 93.4) (width 0.2) (layer "F.Cu") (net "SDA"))
 (segment (start 150.625 91.8) (end 151.025 91.4) (width 0.2) (layer "F.Cu") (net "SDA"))
 (segment (start 156.1 93.1) (end 157 94) (width 0.2) (layer "F.Cu") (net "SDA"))
 (segment (start 153.672057 91.4) (end 154.725 92.452944) (width 0.2) (layer "F.Cu") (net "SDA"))
 (segment (start 157.6 93.4) (end 160.748529 93.4) (width 0.2) (layer "F.Cu") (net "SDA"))
 (segment (start 162 96.693) (end 161.905 96.788) (width 0.2) (layer "F.Cu") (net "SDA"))
 (segment (start 154.725 93.1) (end 156.1 93.1) (width 0.2) (layer "F.Cu") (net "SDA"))
 (segment (start 161.905 94.556471) (end 161.905 96.788) (width 0.2) (layer "F.Cu") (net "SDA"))
 (segment (start 150.625 92.7) (end 150.625 91.8) (width 0.2) (layer "F.Cu") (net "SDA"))
 (segment (start 152.105 93.3) (end 152.105 95.895) (width 0.2) (layer "F.Cu") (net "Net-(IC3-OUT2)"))
 (segment (start 152.155 93.25) (end 152.105 93.3) (width 0.2) (layer "F.Cu") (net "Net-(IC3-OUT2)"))
 (segment (start 155.425 101.225) (end 155.425 100.75) (width 0.2) (layer "F.Cu") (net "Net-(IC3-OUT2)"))
 (segment (start 151.5 101.31005) (end 151.405025 101.405025) (width 0.2) (layer "F.Cu") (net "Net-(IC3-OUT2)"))
 (segment (start 151.5 96.5) (end 151.5 101.31005) (width 0.2) (layer "F.Cu") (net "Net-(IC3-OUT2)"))
 (segment (start 151.894975 102.894975) (end 153.755025 102.894975) (width 0.2) (layer "F.Cu") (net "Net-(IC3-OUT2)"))
 (segment (start 153.755025 102.894975) (end 155.425 101.225) (width 0.2) (layer "F.Cu") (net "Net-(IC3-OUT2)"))
 (segment (start 152.105 95.895) (end 151.5 96.5) (width 0.2) (layer "F.Cu") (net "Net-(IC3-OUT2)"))
 (segment (start 152.74 93.25) (end 152.155 93.25) (width 0.2) (layer "F.Cu") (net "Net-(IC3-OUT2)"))
 (via (at 151.894975 102.894975) (size 0.6) (drill 0.3) (layers "F.Cu" "B.Cu") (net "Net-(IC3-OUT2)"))
 (via (at 151.405025 101.405025) (size 0.6) (drill 0.3) (layers "F.Cu" "B.Cu") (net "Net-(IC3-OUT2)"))
 (segment (start 151.405025 102.405025) (end 151.894975 102.894975) (width 0.2) (layer "B.Cu") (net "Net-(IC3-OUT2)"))
 (segment (start 151.405025 101.405025) (end 151.405025 102.405025) (width 0.2) (layer "B.Cu") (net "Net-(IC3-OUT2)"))
 (segment (start 153.325 92.75) (end 153.5 92.925) (width 0.2) (layer "F.Cu") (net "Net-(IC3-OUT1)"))
 (segment (start 153.5 92.925) (end 153.5 96.5) (width 0.2) (layer "F.Cu") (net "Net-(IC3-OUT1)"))
 (segment (start 154 100) (end 155 100) (width 0.2) (layer "F.Cu") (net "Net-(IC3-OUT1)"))
 (segment (start 153.5 96.5) (end 153.5 99.5) (width 0.2) (layer "F.Cu") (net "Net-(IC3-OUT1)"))
 (segment (start 155 100) (end 155.425 99.575) (width 0.2) (layer "F.Cu") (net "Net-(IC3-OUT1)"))
 (segment (start 152.74 92.75) (end 153.325 92.75) (width 0.2) (layer "F.Cu") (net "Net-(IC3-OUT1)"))
 (segment (start 155.425 99.575) (end 155.425 99.25) (width 0.2) (layer "F.Cu") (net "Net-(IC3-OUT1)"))
 (segment (start 153.5 99.5) (end 154 100) (width 0.2) (layer "F.Cu") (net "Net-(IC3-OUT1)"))
 (segment (start 153.9 92.759314) (end 153.390686 92.25) (width 0.2) (layer "F.Cu") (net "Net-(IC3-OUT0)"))
 (segment (start 154.575 97.425) (end 154.575 99.25) (width 0.2) (layer "F.Cu") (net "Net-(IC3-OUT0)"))
 (segment (start 155.5 96.5) (end 153.9 94.9) (width 0.2) (layer "F.Cu") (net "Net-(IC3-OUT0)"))
 (segment (start 153.9 94.9) (end 153.9 92.759314) (width 0.2) (layer "F.Cu") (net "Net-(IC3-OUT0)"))
 (segment (start 153.390686 92.25) (end 152.74 92.25) (width 0.2) (layer "F.Cu") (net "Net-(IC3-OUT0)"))
 (segment (start 155.5 96.5) (end 154.575 97.425) (width 0.2) (layer "F.Cu") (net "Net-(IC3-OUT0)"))
 (segment (start 144.575379 100.075379) (end 145.575379 100.075379) (width 0.4) (layer "F.Cu") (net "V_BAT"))
 (segment (start 146 100.5) (end 146.45 100.5) (width 0.4) (layer "F.Cu") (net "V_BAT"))
 (segment (start 149.5 104.3) (end 156.7 104.3) (width 0.4) (layer "F.Cu") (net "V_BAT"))
 (segment (start 146.95 101) (end 146.95 101.75) (width 0.4) (layer "F.Cu") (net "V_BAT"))
 (segment (start 145.575379 100.075379) (end 146 100.5) (width 0.4) (layer "F.Cu") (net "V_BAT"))
 (segment (start 153.05 100.75) (end 154.575 100.75) (width 0.4) (layer "F.Cu") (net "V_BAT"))
 (segment (start 156.7 104.3) (end 157 104) (width 0.4) (layer "F.Cu") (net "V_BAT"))
 (segment (start 146.95 101.75) (end 149.5 104.3) (width 0.4) (layer "F.Cu") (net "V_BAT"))
 (segment (start 146.45 100.5) (end 146.95 101) (width 0.4) (layer "F.Cu") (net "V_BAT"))
 (segment (start 149.5 104.3) (end 153.05 100.75) (width 0.4) (layer "F.Cu") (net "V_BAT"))
 (via (at 157 104) (size 0.6) (drill 0.3) (layers "F.Cu" "B.Cu") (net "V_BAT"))
 (via (at 146 100.5) (size 0.6) (drill 0.3) (layers "F.Cu" "B.Cu") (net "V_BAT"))
 (segment (start 157 104) (end 166 104) (width 0.4) (layer "B.Cu") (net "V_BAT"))
 (segment (start 166.45 103.45) (end 166.45 100) (width 0.4) (layer "B.Cu") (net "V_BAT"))
 (segment (start 166 104) (end 166.5 103.5) (width 0.4) (layer "B.Cu") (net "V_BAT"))
 (segment (start 146 100.5) (end 144.05 100.5) (width 0.4) (layer "B.Cu") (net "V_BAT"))
 (segment (start 143.55 100) (end 144 100) (width 0.4) (layer "B.Cu") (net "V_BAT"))
 (segment (start 144.05 100.5) (end 143.55 100) (width 0.4) (layer "B.Cu") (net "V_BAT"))
 (segment (start 166.5 103.5) (end 166.45 103.45) (width 0.4) (layer "B.Cu") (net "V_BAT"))
 (segment (start 154.4945 107.5) (end 147.650758 107.5) (width 0.2) (layer "F.Cu") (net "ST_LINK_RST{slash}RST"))
 (segment (start 158.72 103.2745) (end 154.4945 107.5) (width 0.2) (layer "F.Cu") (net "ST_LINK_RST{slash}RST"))
 (segment (start 158.095 96.788) (end 158.72 97.413) (width 0.2) (layer "F.Cu") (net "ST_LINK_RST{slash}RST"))
 (segment (start 158.72 97.413) (end 158.72 103.2745) (width 0.2) (layer "F.Cu") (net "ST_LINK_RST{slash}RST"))
 (segment (start 162.5 105.7845) (end 162.5 107.5) (width 0.2) (layer "F.Cu") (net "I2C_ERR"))
 (segment (start 159.365 102.212) (end 159.365 102.6495) (width 0.2) (layer "F.Cu") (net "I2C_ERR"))
 (segment (start 159.365 102.6495) (end 162.5 105.7845) (width 0.2) (layer "F.Cu") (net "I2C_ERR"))
 (segment (start 160.635 102.212) (end 160.635 102.6495) (width 0.2) (layer "F.Cu") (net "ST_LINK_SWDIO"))
 (segment (start 160.635 102.6495) (end 161.26 103.2745) (width 0.2) (layer "F.Cu") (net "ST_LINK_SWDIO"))
 (segment (start 162.376258 103.2745) (end 165.575379 100.075379) (width 0.2) (layer "F.Cu") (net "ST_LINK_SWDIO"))
 (segment (start 161.26 103.2745) (end 162.376258 103.2745) (width 0.2) (layer "F.Cu") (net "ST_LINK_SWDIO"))
 (segment (start 163.398026 93.548784) (end 163.398026 100.718974) (width 0.2) (layer "F.Cu") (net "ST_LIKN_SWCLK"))
 (segment (start 163.398026 100.718974) (end 161.905 102.212) (width 0.2) (layer "F.Cu") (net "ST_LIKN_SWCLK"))
 (segment (start 162.5 92.650758) (end 163.398026 93.548784) (width 0.2) (layer "F.Cu") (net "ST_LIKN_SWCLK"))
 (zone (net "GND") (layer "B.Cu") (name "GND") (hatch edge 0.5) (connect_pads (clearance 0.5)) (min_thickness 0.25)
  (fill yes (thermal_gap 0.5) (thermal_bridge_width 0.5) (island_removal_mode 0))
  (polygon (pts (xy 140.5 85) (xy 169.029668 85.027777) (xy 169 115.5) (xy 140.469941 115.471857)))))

